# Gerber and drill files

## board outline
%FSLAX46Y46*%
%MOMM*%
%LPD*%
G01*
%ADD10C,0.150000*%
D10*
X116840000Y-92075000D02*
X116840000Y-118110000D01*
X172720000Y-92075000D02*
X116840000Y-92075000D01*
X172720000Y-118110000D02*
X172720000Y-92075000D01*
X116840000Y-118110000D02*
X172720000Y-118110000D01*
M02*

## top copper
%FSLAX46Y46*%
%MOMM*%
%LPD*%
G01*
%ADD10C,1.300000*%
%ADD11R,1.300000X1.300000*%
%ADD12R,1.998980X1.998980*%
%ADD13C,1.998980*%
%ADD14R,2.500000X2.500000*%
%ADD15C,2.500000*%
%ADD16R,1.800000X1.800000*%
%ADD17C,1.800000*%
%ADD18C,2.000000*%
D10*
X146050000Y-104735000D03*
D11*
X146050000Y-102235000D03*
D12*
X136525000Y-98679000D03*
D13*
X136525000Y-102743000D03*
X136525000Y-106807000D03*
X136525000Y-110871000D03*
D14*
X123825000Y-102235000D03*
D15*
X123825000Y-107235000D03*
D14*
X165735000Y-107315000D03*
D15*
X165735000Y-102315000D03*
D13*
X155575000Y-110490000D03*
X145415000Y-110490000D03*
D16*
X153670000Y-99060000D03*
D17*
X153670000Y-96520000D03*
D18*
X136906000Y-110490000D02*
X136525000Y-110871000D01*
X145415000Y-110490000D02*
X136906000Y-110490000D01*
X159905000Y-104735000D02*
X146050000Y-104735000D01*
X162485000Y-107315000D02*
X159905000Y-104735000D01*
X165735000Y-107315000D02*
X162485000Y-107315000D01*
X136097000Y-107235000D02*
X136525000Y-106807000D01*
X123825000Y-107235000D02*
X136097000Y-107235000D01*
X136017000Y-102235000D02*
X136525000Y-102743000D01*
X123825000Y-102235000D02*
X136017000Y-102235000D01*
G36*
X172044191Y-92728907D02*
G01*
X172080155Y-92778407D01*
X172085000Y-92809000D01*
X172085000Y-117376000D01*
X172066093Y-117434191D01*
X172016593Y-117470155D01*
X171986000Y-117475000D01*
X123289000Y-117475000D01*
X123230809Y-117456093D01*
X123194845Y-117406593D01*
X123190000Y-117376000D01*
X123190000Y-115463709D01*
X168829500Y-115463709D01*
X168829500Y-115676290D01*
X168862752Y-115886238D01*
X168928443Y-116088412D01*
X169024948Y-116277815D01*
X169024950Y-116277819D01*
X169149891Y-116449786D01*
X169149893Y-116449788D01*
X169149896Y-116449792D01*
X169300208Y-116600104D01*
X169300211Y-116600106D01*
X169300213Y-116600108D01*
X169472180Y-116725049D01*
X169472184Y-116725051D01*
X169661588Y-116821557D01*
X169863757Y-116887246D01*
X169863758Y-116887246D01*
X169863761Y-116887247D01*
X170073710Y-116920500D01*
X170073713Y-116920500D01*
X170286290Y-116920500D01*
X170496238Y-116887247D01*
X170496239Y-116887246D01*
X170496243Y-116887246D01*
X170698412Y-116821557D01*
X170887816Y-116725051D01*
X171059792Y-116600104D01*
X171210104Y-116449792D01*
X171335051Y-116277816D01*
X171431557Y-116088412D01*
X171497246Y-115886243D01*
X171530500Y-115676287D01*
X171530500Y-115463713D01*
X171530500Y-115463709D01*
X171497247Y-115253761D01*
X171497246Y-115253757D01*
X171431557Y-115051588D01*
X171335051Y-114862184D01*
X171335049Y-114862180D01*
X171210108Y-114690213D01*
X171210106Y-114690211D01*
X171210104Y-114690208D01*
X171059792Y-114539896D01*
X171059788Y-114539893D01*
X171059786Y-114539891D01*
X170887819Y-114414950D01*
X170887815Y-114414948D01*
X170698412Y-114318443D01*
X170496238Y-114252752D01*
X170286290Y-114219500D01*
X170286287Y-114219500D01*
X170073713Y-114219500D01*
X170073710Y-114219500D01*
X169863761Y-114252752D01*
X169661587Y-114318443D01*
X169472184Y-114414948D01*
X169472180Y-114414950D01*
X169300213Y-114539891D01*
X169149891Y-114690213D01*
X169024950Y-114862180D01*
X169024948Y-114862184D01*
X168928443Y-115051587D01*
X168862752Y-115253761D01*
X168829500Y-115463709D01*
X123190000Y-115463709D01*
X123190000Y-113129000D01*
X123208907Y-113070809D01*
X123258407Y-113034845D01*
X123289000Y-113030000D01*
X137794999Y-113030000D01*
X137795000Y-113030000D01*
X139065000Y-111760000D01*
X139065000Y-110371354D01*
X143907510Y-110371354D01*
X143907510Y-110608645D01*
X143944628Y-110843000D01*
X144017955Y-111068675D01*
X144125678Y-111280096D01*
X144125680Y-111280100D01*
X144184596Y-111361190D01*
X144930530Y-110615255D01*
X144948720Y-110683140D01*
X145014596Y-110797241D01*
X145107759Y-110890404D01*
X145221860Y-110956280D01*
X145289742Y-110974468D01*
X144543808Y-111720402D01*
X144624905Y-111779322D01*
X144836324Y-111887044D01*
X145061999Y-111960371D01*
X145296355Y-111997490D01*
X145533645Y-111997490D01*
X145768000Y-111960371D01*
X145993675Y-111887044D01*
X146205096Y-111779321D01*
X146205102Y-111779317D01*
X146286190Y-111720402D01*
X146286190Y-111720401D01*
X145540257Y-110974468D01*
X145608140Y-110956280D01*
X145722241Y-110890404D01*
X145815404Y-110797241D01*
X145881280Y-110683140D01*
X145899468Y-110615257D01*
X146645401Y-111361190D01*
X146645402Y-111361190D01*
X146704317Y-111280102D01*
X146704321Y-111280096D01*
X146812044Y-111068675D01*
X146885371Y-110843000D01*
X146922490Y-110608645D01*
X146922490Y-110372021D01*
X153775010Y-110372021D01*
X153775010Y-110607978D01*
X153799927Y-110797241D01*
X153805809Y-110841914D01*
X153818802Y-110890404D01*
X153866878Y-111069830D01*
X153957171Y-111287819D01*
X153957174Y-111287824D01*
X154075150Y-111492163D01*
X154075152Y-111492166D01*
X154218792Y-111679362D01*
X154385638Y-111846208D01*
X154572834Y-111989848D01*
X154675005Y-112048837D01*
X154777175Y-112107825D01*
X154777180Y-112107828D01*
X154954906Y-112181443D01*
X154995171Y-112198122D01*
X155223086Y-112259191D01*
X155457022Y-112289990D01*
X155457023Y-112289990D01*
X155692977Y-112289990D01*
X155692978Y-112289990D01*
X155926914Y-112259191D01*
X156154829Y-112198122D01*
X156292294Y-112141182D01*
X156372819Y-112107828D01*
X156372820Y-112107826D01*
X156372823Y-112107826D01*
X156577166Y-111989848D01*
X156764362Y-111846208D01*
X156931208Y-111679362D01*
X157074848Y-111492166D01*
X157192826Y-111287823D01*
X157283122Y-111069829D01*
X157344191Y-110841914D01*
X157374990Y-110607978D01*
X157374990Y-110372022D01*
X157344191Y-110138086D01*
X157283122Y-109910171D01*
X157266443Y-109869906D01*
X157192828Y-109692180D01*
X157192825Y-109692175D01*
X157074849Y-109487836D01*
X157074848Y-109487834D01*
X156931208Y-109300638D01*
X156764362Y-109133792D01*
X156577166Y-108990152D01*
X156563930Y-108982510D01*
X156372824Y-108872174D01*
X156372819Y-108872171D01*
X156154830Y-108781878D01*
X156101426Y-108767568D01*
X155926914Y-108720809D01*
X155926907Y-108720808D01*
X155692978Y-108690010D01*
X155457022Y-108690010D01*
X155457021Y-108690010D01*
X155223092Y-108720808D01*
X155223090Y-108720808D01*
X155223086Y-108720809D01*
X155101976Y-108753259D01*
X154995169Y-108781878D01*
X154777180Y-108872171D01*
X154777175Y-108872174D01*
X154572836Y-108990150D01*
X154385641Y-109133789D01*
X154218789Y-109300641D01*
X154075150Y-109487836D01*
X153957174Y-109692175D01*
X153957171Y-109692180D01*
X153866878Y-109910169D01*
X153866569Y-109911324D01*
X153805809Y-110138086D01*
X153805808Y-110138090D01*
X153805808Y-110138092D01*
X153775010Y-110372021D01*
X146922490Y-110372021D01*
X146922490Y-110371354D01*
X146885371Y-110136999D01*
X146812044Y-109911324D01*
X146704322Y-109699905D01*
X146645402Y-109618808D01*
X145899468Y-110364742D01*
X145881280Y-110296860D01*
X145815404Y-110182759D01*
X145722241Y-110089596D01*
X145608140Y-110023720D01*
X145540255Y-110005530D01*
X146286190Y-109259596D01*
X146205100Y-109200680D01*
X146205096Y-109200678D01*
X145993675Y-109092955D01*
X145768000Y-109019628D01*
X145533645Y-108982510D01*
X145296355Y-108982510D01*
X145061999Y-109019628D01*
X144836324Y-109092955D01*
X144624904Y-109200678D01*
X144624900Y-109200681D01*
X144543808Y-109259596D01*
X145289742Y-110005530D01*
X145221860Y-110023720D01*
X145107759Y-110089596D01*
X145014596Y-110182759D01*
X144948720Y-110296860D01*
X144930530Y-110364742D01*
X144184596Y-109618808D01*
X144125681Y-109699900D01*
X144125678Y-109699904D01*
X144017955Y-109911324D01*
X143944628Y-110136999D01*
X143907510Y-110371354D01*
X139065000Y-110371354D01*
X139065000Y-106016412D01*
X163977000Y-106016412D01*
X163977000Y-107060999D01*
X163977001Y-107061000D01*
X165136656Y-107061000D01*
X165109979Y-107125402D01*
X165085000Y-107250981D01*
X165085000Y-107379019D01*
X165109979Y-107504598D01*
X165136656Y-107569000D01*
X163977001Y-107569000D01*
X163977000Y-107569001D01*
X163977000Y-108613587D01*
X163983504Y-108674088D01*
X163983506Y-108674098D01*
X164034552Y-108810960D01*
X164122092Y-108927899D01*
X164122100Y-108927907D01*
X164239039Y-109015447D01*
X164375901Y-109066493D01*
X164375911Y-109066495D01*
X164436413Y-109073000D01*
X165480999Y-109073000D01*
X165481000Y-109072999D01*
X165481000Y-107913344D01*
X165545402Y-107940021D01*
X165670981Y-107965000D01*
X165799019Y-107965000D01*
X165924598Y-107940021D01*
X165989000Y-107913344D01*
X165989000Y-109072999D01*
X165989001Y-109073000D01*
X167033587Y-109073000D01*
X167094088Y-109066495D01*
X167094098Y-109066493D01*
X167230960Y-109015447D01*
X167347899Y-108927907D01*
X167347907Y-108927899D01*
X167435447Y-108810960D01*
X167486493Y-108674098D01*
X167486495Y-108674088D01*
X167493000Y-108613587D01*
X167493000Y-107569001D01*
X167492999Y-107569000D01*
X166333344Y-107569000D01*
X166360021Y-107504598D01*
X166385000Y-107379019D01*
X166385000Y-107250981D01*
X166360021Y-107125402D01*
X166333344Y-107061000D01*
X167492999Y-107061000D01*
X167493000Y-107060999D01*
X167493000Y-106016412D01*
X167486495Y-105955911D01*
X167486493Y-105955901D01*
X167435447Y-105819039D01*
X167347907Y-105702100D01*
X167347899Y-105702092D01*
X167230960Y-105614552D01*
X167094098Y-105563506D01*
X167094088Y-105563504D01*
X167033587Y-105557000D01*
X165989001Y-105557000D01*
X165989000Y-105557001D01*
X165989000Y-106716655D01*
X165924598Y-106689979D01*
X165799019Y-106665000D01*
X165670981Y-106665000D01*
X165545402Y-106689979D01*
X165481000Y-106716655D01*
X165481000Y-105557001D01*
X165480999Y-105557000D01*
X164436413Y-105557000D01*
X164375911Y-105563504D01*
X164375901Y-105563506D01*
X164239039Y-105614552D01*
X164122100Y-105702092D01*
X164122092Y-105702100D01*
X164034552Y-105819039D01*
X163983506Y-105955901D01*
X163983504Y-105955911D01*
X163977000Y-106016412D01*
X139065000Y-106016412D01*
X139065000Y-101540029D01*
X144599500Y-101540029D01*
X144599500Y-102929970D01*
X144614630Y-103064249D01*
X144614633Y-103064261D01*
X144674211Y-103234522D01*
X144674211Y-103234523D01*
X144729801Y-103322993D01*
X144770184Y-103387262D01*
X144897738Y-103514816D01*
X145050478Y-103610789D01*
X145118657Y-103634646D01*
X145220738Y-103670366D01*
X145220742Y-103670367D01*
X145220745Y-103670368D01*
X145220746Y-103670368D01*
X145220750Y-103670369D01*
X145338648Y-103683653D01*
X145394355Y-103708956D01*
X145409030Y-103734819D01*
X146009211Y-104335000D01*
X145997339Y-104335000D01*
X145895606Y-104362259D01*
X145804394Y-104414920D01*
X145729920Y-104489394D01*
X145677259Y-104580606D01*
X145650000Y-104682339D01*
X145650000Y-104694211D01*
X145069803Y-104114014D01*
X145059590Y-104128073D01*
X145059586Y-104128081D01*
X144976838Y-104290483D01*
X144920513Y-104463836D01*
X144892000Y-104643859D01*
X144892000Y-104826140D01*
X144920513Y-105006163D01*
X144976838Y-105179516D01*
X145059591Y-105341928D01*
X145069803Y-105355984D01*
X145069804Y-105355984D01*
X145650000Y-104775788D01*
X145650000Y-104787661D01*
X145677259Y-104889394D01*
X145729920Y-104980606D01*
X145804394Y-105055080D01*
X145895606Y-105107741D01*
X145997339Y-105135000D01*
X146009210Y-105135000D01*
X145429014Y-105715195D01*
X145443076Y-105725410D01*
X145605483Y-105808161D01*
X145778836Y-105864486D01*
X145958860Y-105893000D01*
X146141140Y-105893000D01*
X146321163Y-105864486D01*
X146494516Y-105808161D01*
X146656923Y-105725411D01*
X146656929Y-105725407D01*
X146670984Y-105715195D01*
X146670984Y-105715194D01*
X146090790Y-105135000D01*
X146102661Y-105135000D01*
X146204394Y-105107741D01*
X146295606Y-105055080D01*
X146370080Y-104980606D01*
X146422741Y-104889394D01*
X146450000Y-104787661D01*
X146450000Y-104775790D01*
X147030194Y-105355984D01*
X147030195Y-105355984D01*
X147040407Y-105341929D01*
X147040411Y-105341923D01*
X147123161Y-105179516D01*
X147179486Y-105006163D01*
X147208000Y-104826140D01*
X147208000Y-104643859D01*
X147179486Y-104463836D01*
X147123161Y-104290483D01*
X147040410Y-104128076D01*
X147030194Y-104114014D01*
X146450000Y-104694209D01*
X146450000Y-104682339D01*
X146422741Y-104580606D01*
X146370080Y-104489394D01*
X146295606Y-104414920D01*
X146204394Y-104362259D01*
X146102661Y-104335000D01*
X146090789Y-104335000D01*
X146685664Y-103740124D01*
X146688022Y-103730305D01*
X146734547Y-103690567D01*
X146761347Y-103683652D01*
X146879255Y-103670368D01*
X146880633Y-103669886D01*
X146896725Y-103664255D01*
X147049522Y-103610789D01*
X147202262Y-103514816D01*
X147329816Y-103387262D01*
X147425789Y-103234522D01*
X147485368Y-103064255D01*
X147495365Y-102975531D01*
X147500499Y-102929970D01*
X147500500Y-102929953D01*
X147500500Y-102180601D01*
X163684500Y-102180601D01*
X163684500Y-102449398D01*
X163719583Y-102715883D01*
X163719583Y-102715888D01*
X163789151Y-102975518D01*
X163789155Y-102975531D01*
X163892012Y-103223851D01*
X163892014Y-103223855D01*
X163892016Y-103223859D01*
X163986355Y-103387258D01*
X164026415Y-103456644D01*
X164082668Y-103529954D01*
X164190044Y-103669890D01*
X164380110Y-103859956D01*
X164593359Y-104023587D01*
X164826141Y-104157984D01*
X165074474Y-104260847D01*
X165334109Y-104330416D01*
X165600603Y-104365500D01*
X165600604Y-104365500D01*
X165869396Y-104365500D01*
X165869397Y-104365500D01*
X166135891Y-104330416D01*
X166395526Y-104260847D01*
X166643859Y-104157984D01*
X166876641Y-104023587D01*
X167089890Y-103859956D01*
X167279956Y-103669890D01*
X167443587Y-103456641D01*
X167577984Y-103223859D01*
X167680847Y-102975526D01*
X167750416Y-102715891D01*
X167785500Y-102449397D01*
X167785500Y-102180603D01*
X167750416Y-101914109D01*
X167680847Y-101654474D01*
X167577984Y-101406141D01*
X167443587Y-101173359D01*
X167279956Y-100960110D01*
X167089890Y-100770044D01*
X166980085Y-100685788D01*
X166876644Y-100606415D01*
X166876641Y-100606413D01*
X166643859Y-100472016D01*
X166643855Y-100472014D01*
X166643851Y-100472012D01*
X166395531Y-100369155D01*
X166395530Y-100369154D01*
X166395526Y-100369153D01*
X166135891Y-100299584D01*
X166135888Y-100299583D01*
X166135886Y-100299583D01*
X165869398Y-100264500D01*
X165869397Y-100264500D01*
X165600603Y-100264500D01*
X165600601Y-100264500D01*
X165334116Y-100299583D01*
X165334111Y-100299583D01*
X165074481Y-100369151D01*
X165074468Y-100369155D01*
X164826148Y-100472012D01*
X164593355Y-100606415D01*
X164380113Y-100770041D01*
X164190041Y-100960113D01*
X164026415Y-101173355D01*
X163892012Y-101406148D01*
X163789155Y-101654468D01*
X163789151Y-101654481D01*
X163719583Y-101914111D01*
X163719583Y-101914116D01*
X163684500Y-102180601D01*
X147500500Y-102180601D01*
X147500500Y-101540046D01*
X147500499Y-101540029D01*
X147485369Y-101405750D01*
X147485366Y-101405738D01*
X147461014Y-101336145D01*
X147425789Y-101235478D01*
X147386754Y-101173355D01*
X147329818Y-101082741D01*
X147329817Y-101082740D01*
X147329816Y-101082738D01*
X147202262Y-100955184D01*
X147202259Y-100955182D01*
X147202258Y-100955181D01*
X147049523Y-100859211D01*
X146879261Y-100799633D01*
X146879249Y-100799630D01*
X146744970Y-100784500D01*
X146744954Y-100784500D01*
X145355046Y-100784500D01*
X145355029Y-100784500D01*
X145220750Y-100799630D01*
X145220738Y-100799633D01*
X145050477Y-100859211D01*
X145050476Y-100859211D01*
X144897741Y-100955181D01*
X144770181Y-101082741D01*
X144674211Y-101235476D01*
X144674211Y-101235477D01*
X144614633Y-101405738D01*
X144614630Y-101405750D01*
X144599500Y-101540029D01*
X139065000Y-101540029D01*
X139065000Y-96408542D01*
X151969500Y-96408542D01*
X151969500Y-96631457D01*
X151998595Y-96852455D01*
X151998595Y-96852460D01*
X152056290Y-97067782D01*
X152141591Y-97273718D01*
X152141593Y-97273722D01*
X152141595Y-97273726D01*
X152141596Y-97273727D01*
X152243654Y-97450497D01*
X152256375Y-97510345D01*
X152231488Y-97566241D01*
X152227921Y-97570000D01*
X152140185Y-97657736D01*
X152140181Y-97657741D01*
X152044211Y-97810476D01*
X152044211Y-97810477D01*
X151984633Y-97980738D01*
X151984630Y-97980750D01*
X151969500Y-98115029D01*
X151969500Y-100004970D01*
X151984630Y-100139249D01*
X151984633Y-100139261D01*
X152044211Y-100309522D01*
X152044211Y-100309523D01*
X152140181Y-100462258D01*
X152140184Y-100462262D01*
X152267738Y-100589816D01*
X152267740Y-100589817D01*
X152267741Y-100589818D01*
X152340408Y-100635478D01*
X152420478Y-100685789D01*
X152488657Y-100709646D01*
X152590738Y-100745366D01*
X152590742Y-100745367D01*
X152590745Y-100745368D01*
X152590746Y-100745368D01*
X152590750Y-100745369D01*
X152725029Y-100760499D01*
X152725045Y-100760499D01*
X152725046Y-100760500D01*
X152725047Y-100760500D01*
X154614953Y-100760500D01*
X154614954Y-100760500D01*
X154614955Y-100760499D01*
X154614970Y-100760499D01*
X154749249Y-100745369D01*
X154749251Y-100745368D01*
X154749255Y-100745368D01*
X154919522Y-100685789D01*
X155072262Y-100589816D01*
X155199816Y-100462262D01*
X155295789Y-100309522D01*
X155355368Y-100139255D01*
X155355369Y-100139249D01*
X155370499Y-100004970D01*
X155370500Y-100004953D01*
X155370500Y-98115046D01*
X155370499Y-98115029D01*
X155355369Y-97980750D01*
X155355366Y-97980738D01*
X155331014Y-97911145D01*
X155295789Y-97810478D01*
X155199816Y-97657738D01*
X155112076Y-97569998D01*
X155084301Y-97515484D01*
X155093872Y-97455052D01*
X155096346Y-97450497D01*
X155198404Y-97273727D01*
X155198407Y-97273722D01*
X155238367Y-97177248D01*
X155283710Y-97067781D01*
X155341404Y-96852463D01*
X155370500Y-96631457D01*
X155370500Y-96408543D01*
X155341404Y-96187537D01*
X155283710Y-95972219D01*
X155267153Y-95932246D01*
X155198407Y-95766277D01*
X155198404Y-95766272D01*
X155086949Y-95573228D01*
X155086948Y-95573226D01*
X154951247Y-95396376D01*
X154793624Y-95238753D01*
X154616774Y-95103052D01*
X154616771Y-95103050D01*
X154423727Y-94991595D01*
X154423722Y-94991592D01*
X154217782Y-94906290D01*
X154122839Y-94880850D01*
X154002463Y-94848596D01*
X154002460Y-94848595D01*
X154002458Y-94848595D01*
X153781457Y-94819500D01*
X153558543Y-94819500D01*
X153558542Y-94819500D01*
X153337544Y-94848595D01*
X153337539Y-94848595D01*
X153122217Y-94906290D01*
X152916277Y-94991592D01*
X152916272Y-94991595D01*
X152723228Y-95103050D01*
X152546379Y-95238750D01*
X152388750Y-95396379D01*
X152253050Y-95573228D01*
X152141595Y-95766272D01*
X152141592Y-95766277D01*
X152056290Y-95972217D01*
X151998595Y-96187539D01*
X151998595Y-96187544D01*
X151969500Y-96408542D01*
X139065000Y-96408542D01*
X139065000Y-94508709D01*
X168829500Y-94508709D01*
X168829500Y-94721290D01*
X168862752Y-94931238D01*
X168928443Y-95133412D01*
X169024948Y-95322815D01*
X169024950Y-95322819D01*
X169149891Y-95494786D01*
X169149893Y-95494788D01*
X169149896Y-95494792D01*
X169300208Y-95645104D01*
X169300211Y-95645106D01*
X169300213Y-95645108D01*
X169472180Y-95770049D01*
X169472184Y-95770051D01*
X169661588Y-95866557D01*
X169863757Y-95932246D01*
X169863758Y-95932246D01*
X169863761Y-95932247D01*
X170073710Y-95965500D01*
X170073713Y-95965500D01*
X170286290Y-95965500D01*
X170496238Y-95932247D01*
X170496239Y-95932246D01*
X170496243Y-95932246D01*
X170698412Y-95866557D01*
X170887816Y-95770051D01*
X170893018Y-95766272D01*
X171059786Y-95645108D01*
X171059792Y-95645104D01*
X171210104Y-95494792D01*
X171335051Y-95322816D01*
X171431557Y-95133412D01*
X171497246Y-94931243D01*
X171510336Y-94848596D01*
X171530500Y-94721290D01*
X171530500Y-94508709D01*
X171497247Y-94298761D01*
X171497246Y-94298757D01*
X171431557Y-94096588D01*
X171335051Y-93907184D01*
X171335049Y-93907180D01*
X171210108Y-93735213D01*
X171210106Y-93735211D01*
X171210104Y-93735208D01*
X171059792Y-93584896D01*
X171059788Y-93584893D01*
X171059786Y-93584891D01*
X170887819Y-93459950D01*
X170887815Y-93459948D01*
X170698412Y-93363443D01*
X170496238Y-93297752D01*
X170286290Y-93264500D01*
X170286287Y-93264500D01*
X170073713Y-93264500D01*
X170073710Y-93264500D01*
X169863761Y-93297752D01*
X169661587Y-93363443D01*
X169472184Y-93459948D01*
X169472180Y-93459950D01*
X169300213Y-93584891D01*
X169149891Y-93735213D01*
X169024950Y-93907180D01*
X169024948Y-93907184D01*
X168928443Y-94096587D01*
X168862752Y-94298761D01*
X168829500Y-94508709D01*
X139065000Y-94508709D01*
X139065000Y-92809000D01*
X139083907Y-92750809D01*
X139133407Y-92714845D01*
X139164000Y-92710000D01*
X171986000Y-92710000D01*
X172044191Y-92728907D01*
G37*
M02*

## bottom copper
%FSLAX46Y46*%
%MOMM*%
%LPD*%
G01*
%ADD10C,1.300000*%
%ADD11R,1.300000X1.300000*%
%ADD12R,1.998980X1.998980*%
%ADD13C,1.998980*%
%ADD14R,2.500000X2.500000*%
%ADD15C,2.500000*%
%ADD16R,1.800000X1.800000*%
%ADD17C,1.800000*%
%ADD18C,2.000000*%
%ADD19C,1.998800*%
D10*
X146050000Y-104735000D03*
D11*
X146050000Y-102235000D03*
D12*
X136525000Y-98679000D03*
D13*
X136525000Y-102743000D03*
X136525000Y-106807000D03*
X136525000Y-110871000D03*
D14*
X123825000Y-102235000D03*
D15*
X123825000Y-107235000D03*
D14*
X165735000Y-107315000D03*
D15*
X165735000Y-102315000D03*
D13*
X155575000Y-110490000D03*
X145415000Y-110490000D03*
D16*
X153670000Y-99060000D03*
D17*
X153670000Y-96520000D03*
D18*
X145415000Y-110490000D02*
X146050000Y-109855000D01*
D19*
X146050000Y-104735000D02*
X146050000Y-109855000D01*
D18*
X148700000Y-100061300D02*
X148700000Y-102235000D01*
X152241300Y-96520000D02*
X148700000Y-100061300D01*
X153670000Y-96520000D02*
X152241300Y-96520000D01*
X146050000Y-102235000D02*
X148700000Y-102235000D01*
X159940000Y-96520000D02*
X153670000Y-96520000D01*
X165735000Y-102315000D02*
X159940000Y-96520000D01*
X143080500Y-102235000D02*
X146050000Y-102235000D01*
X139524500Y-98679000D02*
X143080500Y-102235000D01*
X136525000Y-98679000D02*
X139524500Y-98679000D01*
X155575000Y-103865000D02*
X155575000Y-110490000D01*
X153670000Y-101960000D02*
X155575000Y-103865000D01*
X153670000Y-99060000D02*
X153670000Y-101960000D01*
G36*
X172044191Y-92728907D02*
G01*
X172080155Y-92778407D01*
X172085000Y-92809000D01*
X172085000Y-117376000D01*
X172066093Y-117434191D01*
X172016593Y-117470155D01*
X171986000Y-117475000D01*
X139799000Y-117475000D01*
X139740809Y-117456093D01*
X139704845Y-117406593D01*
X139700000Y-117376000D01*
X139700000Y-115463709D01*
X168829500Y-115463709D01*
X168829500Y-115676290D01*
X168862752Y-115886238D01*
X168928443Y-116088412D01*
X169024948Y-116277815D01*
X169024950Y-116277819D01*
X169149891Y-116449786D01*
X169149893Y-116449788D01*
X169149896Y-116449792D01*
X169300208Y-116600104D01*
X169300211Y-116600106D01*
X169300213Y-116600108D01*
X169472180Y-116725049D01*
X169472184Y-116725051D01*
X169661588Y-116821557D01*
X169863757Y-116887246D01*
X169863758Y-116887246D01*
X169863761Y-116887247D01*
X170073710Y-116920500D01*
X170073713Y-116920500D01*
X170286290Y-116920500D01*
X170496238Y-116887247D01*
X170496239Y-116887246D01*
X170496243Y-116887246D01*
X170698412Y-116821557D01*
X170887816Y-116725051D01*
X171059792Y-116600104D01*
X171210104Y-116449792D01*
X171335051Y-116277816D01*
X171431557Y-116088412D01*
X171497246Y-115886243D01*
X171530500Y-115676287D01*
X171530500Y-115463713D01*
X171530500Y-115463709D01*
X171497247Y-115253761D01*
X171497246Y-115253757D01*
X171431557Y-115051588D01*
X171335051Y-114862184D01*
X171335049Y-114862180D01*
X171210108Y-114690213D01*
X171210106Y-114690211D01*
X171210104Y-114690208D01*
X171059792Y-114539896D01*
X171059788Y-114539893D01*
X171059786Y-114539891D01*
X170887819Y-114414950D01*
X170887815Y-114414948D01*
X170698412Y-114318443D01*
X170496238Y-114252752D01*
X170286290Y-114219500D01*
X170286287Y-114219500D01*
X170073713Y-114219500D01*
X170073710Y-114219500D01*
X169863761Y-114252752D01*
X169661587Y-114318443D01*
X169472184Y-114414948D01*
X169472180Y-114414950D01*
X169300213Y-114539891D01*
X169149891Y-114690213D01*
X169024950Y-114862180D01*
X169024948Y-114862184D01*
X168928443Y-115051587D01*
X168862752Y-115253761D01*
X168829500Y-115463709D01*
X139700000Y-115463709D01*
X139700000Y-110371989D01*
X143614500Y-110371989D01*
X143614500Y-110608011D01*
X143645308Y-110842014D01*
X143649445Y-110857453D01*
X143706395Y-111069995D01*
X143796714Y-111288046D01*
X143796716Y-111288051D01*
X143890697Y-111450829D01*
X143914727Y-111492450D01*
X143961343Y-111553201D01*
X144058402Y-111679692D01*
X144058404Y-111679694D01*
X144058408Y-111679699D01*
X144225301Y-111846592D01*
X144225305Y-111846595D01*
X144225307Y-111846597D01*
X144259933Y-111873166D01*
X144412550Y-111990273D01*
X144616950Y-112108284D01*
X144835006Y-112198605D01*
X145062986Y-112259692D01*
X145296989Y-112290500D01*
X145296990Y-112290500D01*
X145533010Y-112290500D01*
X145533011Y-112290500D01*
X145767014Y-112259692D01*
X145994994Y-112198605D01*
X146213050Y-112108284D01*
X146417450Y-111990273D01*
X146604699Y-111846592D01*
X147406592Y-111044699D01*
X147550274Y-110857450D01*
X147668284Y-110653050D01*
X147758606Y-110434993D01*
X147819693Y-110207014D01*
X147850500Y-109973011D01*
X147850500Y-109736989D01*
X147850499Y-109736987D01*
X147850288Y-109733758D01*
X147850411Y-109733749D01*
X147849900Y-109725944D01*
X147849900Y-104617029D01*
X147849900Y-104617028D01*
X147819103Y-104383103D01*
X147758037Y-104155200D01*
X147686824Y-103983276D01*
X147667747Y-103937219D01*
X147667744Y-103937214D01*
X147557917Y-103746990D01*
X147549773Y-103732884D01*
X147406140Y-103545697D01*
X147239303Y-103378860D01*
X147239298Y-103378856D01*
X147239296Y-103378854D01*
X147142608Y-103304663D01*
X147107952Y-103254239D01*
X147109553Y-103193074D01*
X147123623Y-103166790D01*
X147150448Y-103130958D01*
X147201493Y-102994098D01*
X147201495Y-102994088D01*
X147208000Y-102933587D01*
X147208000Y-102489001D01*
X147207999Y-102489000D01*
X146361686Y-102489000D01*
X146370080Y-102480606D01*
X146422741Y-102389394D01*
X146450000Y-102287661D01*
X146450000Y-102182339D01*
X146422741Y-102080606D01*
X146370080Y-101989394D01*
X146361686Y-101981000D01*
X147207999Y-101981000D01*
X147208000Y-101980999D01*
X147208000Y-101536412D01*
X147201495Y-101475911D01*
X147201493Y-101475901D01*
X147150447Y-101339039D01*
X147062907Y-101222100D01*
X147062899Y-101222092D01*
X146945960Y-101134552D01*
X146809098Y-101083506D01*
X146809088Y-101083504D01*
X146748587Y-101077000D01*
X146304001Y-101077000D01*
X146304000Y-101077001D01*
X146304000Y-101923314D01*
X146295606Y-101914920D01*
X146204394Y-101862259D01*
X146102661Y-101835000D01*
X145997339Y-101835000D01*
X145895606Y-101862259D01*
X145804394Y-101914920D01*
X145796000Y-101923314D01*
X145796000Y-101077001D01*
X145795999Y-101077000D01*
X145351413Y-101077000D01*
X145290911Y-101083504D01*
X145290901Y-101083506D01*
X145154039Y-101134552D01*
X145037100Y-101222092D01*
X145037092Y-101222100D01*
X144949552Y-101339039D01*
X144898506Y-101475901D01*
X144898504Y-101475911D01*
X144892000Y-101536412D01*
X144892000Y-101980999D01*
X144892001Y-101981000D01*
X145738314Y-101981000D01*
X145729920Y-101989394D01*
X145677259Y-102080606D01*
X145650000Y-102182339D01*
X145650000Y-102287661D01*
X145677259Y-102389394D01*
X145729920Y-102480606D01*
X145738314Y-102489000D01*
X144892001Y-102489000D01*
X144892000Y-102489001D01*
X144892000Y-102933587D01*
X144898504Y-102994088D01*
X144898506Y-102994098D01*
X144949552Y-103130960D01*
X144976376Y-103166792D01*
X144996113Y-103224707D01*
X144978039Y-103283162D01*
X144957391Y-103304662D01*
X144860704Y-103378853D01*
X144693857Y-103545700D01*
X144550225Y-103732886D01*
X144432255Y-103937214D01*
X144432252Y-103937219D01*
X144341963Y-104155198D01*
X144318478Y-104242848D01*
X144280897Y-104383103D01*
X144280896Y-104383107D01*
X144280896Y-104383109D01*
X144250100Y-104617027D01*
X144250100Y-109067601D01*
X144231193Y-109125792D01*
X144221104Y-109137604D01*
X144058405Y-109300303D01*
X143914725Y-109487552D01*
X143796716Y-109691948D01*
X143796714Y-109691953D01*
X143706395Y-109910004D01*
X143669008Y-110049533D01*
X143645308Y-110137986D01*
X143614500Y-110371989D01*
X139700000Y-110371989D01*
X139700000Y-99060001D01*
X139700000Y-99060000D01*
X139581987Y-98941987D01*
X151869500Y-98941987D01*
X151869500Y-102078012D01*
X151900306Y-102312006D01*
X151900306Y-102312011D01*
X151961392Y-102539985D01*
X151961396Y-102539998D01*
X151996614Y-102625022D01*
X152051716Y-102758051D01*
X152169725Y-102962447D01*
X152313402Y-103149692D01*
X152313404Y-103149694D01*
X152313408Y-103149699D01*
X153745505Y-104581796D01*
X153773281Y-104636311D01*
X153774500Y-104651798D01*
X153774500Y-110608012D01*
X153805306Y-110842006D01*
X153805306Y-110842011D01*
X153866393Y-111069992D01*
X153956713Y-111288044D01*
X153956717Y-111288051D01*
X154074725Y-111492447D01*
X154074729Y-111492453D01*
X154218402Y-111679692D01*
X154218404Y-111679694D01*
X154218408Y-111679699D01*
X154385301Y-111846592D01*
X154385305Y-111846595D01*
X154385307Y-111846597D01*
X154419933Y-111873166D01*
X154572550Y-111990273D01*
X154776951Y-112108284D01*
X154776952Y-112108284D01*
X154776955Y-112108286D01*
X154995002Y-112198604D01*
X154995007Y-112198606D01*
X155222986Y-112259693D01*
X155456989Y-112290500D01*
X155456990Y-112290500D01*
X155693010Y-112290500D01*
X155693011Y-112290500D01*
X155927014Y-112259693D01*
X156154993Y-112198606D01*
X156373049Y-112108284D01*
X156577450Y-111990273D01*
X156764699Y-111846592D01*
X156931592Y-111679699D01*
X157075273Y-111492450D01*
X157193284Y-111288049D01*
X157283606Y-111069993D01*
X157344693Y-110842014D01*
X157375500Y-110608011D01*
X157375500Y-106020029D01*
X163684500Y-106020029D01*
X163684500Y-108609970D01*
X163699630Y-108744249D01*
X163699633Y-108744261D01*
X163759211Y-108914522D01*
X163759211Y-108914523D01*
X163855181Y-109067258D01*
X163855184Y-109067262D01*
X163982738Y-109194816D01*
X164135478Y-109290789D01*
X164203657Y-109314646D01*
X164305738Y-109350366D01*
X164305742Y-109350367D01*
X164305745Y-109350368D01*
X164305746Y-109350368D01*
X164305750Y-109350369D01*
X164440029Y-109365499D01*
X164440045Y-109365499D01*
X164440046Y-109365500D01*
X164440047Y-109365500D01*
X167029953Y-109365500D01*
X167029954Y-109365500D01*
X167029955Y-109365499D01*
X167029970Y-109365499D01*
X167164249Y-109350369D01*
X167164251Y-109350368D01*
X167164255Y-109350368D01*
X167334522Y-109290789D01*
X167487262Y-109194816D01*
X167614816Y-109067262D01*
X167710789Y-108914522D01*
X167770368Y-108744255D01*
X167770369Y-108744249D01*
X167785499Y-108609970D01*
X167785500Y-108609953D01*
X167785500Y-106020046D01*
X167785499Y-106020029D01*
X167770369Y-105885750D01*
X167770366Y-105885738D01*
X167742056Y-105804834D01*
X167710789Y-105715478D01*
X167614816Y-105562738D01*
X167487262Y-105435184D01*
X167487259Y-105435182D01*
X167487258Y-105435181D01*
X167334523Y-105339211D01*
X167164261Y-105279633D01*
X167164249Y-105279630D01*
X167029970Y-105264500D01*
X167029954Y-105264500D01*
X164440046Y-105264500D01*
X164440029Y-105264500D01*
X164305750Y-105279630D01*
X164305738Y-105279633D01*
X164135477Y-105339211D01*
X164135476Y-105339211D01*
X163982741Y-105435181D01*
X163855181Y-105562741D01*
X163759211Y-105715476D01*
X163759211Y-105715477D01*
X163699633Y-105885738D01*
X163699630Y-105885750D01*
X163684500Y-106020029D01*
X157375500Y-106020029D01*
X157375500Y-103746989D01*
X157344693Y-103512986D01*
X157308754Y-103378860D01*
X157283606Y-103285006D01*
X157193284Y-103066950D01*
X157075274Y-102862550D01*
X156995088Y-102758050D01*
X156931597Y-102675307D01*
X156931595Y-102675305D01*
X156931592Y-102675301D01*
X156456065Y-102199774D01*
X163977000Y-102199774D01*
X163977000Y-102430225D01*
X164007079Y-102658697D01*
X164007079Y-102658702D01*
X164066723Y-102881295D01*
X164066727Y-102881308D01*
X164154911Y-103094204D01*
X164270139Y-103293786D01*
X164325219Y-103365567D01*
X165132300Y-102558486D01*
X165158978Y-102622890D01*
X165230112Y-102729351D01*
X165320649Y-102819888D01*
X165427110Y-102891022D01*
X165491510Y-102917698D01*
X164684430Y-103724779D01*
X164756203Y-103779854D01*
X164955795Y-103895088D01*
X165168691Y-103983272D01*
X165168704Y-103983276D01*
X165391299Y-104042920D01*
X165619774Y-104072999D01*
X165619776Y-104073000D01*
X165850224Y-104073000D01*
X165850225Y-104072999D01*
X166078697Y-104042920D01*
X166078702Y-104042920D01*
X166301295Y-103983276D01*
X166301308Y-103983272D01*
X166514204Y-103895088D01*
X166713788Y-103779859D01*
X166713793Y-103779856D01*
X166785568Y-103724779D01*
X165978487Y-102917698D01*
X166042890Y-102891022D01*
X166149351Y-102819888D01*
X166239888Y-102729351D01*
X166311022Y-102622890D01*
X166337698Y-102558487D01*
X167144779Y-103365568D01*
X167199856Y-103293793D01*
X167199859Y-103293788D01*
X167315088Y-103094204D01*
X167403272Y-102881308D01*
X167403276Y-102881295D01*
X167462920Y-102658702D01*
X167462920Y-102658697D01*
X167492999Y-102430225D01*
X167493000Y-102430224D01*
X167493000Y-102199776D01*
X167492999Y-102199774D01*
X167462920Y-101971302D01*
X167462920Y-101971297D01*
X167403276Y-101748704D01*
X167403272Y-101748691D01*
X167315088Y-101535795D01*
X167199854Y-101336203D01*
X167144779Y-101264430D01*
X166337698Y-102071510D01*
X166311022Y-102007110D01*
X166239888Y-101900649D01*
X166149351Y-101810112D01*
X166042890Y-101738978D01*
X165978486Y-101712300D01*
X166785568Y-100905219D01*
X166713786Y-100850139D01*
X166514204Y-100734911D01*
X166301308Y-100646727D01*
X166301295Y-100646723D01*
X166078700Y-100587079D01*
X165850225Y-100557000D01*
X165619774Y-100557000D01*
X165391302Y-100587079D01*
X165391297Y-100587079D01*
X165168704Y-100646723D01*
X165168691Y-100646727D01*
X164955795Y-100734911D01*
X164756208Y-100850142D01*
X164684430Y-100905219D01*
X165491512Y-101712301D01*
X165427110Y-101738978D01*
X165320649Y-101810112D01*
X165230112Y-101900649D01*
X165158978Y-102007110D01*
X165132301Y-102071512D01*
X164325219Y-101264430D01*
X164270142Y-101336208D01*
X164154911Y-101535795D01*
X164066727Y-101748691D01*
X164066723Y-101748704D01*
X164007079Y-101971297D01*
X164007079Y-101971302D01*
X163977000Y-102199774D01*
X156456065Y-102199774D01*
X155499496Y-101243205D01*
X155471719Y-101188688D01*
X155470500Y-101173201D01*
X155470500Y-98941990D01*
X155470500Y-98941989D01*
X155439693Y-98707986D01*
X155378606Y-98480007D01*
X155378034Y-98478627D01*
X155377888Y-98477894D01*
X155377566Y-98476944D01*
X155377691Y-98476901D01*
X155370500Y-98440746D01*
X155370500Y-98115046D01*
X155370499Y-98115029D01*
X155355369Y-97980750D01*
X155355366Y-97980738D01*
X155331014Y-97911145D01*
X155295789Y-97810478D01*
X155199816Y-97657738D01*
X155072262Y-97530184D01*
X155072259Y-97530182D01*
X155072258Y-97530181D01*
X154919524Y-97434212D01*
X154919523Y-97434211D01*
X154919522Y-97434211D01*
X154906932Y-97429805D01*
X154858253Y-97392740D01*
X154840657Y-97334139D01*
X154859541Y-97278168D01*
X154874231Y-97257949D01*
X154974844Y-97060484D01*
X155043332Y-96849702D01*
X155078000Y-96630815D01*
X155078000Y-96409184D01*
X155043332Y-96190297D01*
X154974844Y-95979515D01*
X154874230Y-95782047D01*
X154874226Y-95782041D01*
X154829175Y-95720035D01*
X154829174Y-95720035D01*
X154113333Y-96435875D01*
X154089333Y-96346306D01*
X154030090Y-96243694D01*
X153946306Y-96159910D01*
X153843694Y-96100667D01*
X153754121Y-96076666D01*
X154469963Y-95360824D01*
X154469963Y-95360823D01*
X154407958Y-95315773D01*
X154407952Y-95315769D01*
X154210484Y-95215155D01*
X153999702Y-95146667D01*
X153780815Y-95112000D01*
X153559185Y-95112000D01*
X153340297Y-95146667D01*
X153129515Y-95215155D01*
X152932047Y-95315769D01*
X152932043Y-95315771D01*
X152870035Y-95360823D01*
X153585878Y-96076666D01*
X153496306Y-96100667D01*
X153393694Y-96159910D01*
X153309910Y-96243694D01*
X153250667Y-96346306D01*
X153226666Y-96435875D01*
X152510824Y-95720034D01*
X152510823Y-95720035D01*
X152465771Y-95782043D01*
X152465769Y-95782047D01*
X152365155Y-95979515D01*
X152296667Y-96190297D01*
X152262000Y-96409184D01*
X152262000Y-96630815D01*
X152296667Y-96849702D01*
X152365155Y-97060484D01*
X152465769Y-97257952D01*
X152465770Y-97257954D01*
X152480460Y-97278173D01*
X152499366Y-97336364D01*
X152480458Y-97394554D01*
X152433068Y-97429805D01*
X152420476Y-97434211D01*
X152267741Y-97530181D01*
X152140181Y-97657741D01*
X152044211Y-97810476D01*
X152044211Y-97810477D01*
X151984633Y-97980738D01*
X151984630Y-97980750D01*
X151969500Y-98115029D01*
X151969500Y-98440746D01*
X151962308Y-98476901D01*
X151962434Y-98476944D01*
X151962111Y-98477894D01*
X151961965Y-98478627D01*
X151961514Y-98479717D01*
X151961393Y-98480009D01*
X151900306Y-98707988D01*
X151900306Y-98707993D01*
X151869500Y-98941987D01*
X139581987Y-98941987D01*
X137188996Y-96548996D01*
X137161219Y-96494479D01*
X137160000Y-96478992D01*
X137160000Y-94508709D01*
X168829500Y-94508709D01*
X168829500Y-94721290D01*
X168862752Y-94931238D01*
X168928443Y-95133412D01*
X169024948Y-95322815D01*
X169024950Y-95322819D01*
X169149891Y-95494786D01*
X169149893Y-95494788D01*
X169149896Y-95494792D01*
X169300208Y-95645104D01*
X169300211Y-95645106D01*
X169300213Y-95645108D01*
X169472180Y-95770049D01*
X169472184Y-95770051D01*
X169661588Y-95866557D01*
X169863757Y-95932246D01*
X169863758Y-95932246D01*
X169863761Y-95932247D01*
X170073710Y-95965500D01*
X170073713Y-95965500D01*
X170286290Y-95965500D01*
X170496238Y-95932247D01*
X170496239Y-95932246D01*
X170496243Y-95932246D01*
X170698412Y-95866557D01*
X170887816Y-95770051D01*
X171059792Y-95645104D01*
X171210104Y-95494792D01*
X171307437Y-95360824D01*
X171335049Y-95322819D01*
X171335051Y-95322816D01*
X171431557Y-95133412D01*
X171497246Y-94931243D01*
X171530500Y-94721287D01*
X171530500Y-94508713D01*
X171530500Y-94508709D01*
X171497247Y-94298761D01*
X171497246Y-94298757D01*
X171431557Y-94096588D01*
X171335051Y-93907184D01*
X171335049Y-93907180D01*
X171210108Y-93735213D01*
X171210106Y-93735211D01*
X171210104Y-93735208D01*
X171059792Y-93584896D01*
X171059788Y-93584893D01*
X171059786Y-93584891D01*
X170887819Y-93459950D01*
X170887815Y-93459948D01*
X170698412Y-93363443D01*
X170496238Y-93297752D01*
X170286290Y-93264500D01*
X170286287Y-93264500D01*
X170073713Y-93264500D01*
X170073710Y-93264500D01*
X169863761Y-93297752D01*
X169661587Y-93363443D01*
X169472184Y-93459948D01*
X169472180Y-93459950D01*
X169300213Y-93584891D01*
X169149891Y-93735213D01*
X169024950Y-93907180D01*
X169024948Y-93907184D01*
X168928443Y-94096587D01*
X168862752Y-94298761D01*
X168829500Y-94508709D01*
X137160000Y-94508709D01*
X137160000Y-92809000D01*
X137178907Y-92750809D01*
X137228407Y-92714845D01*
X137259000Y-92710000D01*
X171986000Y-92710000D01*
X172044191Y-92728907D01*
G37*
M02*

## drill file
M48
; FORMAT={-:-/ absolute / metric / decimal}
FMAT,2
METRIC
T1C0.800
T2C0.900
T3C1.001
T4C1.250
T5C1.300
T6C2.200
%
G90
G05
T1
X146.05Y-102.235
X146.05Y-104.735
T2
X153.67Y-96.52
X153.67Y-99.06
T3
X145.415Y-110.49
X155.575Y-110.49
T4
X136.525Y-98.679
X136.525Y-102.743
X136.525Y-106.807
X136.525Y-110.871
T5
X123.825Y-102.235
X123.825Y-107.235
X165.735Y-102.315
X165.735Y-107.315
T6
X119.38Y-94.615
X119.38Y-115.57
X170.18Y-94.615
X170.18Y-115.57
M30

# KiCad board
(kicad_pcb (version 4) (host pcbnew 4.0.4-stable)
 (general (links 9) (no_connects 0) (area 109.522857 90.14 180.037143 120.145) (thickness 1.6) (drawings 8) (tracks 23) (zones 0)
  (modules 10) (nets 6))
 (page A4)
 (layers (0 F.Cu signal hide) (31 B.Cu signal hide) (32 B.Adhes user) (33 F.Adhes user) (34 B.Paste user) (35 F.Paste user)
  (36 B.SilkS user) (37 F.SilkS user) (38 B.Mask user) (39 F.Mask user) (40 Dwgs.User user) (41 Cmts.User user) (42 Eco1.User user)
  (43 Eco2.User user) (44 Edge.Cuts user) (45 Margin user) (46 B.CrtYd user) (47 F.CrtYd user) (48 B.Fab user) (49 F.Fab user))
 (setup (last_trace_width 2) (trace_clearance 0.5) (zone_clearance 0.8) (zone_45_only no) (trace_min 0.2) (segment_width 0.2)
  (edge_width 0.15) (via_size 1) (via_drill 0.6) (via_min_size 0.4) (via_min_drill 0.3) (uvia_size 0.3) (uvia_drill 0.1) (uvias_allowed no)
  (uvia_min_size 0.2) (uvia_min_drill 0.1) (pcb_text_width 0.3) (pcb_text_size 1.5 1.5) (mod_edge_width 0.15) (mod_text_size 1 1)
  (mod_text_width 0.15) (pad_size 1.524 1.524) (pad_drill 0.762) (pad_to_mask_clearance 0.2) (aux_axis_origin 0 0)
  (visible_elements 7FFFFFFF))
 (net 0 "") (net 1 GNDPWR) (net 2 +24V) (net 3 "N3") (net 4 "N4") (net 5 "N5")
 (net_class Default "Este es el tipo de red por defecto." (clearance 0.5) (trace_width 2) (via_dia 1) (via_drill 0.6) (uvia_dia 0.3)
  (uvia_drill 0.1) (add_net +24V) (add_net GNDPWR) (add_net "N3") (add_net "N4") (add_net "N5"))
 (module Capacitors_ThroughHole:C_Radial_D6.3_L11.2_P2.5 (layer F.Cu) (at 146.05 102.235 270)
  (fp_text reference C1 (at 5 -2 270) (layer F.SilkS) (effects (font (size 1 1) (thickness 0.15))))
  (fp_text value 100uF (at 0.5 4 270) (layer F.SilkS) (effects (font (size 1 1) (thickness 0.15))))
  (pad 2 thru_hole circle (at 2.5 0 270) (size 1.3 1.3) (drill 0.8) (layers *.Cu *.Mask F.SilkS) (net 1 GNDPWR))
  (pad 1 thru_hole rect (at 0 0 270) (size 1.3 1.3) (drill 0.8) (layers *.Cu *.Mask F.SilkS) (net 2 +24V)))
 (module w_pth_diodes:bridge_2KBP (layer F.Cu) (at 136.525 104.775 270)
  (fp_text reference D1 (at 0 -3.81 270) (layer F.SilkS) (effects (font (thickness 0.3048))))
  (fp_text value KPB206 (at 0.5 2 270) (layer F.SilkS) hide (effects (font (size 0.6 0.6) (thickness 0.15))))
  (pad 1 thru_hole rect (at -6.096 0 270) (size 1.99898 1.99898) (drill 1.24968) (layers *.Cu *.Mask F.SilkS) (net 2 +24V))
  (pad 2 thru_hole circle (at -2.032 0 270) (size 1.99898 1.99898) (drill 1.24968) (layers *.Cu *.Mask F.SilkS) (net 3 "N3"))
  (pad 3 thru_hole circle (at 2.032 0 270) (size 1.99898 1.99898) (drill 1.24968) (layers *.Cu *.Mask F.SilkS) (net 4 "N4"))
  (pad 4 thru_hole circle (at 6.096 0 270) (size 1.99898 1.99898) (drill 1.24968) (layers *.Cu *.Mask F.SilkS) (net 1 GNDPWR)))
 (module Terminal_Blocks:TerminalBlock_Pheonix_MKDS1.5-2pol (layer F.Cu) (at 123.825 102.235 270)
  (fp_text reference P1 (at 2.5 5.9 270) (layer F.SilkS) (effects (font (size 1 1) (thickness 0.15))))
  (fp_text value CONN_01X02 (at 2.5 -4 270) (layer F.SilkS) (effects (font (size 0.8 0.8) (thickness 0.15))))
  (pad 1 thru_hole rect (at 0 0 270) (size 2.5 2.5) (drill 1.3) (layers *.Cu *.Mask F.SilkS) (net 3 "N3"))
  (pad 2 thru_hole circle (at 5 0 270) (size 2.5 2.5) (drill 1.3) (layers *.Cu *.Mask F.SilkS) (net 4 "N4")))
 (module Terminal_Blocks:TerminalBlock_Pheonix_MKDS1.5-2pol (layer F.Cu) (at 165.735 107.315 90)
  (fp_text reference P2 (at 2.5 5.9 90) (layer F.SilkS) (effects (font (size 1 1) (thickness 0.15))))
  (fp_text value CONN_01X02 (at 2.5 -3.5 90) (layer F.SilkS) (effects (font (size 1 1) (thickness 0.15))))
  (pad 1 thru_hole rect (at 0 0 90) (size 2.5 2.5) (drill 1.3) (layers *.Cu *.Mask F.SilkS) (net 1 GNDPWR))
  (pad 2 thru_hole circle (at 5 0 90) (size 2.5 2.5) (drill 1.3) (layers *.Cu *.Mask F.SilkS) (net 2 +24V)))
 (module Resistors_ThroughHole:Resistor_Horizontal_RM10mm (layer F.Cu) (at 155.575 110.49 180)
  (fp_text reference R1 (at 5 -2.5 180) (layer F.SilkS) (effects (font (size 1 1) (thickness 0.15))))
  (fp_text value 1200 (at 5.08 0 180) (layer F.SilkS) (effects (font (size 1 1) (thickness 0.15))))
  (pad 1 thru_hole circle (at 0 0 180) (size 1.99898 1.99898) (drill 1.00076) (layers *.Cu *.SilkS *.Mask) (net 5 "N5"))
  (pad 2 thru_hole circle (at 10.16 0 180) (size 1.99898 1.99898) (drill 1.00076) (layers *.Cu *.SilkS *.Mask) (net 1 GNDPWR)))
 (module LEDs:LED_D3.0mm (layer F.Cu) (at 153.67 99.06 90)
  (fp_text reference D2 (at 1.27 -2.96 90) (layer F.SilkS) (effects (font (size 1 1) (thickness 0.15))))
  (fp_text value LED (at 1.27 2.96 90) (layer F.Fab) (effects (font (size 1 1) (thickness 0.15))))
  (pad 1 thru_hole rect (at 0 0 90) (size 1.8 1.8) (drill 0.9) (layers *.Cu *.Mask) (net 5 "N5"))
  (pad 2 thru_hole circle (at 2.54 0 90) (size 1.8 1.8) (drill 0.9) (layers *.Cu *.Mask) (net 2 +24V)))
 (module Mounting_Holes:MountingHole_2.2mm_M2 (layer F.Cu) (at 119.38 94.615)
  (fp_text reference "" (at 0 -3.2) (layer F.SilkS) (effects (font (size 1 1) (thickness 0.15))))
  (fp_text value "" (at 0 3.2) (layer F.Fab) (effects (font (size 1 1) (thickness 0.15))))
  (pad 1 np_thru_hole circle (at 0 0) (size 2.2 2.2) (drill 2.2) (layers *.Cu *.Mask)))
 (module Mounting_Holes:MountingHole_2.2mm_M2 (layer F.Cu) (at 119.38 115.57)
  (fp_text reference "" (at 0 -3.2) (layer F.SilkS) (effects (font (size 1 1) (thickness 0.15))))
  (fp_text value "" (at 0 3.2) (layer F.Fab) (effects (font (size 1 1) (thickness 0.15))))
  (pad 1 np_thru_hole circle (at 0 0) (size 2.2 2.2) (drill 2.2) (layers *.Cu *.Mask)))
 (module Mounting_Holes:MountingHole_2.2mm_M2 (layer F.Cu) (at 170.18 94.615)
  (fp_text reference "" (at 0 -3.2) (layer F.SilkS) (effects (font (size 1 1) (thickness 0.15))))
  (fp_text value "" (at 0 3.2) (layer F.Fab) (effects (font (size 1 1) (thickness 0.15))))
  (pad 1 np_thru_hole circle (at 0 0) (size 2.2 2.2) (drill 2.2) (layers *.Cu *.Mask)))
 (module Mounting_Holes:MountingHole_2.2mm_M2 (layer F.Cu) (at 170.18 115.57)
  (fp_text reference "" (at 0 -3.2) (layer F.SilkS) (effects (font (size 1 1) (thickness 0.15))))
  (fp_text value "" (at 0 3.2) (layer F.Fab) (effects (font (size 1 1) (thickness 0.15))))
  (pad 1 np_thru_hole circle (at 0 0) (size 2.2 2.2) (drill 2.2) (layers *.Cu *.Mask)))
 (gr_line (start 116.84 92.075) (end 116.84 118.11) (angle 90) (layer Edge.Cuts) (width 0.15))
 (gr_line (start 172.72 92.075) (end 116.84 92.075) (angle 90) (layer Edge.Cuts) (width 0.15))
 (gr_line (start 172.72 118.11) (end 172.72 92.075) (angle 90) (layer Edge.Cuts) (width 0.15))
 (gr_line (start 116.84 118.11) (end 172.72 118.11) (angle 90) (layer Edge.Cuts) (width 0.15))
 (segment (start 136.906 110.49) (end 136.525 110.871) (width 2) (layer F.Cu) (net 1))
 (segment (start 145.415 110.49) (end 136.906 110.49) (width 2) (layer F.Cu) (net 1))
 (segment (start 159.905 104.735) (end 146.05 104.735) (width 2) (layer F.Cu) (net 1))
 (segment (start 162.485 107.315) (end 159.905 104.735) (width 2) (layer F.Cu) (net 1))
 (segment (start 165.735 107.315) (end 162.485 107.315) (width 2) (layer F.Cu) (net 1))
 (segment (start 145.415 110.49) (end 146.05 109.855) (width 2) (layer B.Cu) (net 1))
 (segment (start 146.05 104.735) (end 146.05 109.855) (width 1.9988) (layer B.Cu) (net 1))
 (segment (start 148.7 100.0613) (end 148.7 102.235) (width 2) (layer B.Cu) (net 2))
 (segment (start 152.2413 96.52) (end 148.7 100.0613) (width 2) (layer B.Cu) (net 2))
 (segment (start 153.67 96.52) (end 152.2413 96.52) (width 2) (layer B.Cu) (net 2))
 (segment (start 146.05 102.235) (end 148.7 102.235) (width 2) (layer B.Cu) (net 2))
 (segment (start 159.94 96.52) (end 153.67 96.52) (width 2) (layer B.Cu) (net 2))
 (segment (start 165.735 102.315) (end 159.94 96.52) (width 2) (layer B.Cu) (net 2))
 (segment (start 143.0805 102.235) (end 146.05 102.235) (width 2) (layer B.Cu) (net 2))
 (segment (start 139.5245 98.679) (end 143.0805 102.235) (width 2) (layer B.Cu) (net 2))
 (segment (start 136.525 98.679) (end 139.5245 98.679) (width 2) (layer B.Cu) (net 2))
 (segment (start 136.097 107.235) (end 136.525 106.807) (width 2) (layer F.Cu) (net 4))
 (segment (start 123.825 107.235) (end 136.097 107.235) (width 2) (layer F.Cu) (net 4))
 (segment (start 155.575 103.865) (end 155.575 110.49) (width 2) (layer B.Cu) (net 5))
 (segment (start 153.67 101.96) (end 155.575 103.865) (width 2) (layer B.Cu) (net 5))
 (segment (start 153.67 99.06) (end 153.67 101.96) (width 2) (layer B.Cu) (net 5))
 (segment (start 136.017 102.235) (end 136.525 102.743) (width 2) (layer F.Cu) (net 3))
 (segment (start 123.825 102.235) (end 136.017 102.235) (width 2) (layer F.Cu) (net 3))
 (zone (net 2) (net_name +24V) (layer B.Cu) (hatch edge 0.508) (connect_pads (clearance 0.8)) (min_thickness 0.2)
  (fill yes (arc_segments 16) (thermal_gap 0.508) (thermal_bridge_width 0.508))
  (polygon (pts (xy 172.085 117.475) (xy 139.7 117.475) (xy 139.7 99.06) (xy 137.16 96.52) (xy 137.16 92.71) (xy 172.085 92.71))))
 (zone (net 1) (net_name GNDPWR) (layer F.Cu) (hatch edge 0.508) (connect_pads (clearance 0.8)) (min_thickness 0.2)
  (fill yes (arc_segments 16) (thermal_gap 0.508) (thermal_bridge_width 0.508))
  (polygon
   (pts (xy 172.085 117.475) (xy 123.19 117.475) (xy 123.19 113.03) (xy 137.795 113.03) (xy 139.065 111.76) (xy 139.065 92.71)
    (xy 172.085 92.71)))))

